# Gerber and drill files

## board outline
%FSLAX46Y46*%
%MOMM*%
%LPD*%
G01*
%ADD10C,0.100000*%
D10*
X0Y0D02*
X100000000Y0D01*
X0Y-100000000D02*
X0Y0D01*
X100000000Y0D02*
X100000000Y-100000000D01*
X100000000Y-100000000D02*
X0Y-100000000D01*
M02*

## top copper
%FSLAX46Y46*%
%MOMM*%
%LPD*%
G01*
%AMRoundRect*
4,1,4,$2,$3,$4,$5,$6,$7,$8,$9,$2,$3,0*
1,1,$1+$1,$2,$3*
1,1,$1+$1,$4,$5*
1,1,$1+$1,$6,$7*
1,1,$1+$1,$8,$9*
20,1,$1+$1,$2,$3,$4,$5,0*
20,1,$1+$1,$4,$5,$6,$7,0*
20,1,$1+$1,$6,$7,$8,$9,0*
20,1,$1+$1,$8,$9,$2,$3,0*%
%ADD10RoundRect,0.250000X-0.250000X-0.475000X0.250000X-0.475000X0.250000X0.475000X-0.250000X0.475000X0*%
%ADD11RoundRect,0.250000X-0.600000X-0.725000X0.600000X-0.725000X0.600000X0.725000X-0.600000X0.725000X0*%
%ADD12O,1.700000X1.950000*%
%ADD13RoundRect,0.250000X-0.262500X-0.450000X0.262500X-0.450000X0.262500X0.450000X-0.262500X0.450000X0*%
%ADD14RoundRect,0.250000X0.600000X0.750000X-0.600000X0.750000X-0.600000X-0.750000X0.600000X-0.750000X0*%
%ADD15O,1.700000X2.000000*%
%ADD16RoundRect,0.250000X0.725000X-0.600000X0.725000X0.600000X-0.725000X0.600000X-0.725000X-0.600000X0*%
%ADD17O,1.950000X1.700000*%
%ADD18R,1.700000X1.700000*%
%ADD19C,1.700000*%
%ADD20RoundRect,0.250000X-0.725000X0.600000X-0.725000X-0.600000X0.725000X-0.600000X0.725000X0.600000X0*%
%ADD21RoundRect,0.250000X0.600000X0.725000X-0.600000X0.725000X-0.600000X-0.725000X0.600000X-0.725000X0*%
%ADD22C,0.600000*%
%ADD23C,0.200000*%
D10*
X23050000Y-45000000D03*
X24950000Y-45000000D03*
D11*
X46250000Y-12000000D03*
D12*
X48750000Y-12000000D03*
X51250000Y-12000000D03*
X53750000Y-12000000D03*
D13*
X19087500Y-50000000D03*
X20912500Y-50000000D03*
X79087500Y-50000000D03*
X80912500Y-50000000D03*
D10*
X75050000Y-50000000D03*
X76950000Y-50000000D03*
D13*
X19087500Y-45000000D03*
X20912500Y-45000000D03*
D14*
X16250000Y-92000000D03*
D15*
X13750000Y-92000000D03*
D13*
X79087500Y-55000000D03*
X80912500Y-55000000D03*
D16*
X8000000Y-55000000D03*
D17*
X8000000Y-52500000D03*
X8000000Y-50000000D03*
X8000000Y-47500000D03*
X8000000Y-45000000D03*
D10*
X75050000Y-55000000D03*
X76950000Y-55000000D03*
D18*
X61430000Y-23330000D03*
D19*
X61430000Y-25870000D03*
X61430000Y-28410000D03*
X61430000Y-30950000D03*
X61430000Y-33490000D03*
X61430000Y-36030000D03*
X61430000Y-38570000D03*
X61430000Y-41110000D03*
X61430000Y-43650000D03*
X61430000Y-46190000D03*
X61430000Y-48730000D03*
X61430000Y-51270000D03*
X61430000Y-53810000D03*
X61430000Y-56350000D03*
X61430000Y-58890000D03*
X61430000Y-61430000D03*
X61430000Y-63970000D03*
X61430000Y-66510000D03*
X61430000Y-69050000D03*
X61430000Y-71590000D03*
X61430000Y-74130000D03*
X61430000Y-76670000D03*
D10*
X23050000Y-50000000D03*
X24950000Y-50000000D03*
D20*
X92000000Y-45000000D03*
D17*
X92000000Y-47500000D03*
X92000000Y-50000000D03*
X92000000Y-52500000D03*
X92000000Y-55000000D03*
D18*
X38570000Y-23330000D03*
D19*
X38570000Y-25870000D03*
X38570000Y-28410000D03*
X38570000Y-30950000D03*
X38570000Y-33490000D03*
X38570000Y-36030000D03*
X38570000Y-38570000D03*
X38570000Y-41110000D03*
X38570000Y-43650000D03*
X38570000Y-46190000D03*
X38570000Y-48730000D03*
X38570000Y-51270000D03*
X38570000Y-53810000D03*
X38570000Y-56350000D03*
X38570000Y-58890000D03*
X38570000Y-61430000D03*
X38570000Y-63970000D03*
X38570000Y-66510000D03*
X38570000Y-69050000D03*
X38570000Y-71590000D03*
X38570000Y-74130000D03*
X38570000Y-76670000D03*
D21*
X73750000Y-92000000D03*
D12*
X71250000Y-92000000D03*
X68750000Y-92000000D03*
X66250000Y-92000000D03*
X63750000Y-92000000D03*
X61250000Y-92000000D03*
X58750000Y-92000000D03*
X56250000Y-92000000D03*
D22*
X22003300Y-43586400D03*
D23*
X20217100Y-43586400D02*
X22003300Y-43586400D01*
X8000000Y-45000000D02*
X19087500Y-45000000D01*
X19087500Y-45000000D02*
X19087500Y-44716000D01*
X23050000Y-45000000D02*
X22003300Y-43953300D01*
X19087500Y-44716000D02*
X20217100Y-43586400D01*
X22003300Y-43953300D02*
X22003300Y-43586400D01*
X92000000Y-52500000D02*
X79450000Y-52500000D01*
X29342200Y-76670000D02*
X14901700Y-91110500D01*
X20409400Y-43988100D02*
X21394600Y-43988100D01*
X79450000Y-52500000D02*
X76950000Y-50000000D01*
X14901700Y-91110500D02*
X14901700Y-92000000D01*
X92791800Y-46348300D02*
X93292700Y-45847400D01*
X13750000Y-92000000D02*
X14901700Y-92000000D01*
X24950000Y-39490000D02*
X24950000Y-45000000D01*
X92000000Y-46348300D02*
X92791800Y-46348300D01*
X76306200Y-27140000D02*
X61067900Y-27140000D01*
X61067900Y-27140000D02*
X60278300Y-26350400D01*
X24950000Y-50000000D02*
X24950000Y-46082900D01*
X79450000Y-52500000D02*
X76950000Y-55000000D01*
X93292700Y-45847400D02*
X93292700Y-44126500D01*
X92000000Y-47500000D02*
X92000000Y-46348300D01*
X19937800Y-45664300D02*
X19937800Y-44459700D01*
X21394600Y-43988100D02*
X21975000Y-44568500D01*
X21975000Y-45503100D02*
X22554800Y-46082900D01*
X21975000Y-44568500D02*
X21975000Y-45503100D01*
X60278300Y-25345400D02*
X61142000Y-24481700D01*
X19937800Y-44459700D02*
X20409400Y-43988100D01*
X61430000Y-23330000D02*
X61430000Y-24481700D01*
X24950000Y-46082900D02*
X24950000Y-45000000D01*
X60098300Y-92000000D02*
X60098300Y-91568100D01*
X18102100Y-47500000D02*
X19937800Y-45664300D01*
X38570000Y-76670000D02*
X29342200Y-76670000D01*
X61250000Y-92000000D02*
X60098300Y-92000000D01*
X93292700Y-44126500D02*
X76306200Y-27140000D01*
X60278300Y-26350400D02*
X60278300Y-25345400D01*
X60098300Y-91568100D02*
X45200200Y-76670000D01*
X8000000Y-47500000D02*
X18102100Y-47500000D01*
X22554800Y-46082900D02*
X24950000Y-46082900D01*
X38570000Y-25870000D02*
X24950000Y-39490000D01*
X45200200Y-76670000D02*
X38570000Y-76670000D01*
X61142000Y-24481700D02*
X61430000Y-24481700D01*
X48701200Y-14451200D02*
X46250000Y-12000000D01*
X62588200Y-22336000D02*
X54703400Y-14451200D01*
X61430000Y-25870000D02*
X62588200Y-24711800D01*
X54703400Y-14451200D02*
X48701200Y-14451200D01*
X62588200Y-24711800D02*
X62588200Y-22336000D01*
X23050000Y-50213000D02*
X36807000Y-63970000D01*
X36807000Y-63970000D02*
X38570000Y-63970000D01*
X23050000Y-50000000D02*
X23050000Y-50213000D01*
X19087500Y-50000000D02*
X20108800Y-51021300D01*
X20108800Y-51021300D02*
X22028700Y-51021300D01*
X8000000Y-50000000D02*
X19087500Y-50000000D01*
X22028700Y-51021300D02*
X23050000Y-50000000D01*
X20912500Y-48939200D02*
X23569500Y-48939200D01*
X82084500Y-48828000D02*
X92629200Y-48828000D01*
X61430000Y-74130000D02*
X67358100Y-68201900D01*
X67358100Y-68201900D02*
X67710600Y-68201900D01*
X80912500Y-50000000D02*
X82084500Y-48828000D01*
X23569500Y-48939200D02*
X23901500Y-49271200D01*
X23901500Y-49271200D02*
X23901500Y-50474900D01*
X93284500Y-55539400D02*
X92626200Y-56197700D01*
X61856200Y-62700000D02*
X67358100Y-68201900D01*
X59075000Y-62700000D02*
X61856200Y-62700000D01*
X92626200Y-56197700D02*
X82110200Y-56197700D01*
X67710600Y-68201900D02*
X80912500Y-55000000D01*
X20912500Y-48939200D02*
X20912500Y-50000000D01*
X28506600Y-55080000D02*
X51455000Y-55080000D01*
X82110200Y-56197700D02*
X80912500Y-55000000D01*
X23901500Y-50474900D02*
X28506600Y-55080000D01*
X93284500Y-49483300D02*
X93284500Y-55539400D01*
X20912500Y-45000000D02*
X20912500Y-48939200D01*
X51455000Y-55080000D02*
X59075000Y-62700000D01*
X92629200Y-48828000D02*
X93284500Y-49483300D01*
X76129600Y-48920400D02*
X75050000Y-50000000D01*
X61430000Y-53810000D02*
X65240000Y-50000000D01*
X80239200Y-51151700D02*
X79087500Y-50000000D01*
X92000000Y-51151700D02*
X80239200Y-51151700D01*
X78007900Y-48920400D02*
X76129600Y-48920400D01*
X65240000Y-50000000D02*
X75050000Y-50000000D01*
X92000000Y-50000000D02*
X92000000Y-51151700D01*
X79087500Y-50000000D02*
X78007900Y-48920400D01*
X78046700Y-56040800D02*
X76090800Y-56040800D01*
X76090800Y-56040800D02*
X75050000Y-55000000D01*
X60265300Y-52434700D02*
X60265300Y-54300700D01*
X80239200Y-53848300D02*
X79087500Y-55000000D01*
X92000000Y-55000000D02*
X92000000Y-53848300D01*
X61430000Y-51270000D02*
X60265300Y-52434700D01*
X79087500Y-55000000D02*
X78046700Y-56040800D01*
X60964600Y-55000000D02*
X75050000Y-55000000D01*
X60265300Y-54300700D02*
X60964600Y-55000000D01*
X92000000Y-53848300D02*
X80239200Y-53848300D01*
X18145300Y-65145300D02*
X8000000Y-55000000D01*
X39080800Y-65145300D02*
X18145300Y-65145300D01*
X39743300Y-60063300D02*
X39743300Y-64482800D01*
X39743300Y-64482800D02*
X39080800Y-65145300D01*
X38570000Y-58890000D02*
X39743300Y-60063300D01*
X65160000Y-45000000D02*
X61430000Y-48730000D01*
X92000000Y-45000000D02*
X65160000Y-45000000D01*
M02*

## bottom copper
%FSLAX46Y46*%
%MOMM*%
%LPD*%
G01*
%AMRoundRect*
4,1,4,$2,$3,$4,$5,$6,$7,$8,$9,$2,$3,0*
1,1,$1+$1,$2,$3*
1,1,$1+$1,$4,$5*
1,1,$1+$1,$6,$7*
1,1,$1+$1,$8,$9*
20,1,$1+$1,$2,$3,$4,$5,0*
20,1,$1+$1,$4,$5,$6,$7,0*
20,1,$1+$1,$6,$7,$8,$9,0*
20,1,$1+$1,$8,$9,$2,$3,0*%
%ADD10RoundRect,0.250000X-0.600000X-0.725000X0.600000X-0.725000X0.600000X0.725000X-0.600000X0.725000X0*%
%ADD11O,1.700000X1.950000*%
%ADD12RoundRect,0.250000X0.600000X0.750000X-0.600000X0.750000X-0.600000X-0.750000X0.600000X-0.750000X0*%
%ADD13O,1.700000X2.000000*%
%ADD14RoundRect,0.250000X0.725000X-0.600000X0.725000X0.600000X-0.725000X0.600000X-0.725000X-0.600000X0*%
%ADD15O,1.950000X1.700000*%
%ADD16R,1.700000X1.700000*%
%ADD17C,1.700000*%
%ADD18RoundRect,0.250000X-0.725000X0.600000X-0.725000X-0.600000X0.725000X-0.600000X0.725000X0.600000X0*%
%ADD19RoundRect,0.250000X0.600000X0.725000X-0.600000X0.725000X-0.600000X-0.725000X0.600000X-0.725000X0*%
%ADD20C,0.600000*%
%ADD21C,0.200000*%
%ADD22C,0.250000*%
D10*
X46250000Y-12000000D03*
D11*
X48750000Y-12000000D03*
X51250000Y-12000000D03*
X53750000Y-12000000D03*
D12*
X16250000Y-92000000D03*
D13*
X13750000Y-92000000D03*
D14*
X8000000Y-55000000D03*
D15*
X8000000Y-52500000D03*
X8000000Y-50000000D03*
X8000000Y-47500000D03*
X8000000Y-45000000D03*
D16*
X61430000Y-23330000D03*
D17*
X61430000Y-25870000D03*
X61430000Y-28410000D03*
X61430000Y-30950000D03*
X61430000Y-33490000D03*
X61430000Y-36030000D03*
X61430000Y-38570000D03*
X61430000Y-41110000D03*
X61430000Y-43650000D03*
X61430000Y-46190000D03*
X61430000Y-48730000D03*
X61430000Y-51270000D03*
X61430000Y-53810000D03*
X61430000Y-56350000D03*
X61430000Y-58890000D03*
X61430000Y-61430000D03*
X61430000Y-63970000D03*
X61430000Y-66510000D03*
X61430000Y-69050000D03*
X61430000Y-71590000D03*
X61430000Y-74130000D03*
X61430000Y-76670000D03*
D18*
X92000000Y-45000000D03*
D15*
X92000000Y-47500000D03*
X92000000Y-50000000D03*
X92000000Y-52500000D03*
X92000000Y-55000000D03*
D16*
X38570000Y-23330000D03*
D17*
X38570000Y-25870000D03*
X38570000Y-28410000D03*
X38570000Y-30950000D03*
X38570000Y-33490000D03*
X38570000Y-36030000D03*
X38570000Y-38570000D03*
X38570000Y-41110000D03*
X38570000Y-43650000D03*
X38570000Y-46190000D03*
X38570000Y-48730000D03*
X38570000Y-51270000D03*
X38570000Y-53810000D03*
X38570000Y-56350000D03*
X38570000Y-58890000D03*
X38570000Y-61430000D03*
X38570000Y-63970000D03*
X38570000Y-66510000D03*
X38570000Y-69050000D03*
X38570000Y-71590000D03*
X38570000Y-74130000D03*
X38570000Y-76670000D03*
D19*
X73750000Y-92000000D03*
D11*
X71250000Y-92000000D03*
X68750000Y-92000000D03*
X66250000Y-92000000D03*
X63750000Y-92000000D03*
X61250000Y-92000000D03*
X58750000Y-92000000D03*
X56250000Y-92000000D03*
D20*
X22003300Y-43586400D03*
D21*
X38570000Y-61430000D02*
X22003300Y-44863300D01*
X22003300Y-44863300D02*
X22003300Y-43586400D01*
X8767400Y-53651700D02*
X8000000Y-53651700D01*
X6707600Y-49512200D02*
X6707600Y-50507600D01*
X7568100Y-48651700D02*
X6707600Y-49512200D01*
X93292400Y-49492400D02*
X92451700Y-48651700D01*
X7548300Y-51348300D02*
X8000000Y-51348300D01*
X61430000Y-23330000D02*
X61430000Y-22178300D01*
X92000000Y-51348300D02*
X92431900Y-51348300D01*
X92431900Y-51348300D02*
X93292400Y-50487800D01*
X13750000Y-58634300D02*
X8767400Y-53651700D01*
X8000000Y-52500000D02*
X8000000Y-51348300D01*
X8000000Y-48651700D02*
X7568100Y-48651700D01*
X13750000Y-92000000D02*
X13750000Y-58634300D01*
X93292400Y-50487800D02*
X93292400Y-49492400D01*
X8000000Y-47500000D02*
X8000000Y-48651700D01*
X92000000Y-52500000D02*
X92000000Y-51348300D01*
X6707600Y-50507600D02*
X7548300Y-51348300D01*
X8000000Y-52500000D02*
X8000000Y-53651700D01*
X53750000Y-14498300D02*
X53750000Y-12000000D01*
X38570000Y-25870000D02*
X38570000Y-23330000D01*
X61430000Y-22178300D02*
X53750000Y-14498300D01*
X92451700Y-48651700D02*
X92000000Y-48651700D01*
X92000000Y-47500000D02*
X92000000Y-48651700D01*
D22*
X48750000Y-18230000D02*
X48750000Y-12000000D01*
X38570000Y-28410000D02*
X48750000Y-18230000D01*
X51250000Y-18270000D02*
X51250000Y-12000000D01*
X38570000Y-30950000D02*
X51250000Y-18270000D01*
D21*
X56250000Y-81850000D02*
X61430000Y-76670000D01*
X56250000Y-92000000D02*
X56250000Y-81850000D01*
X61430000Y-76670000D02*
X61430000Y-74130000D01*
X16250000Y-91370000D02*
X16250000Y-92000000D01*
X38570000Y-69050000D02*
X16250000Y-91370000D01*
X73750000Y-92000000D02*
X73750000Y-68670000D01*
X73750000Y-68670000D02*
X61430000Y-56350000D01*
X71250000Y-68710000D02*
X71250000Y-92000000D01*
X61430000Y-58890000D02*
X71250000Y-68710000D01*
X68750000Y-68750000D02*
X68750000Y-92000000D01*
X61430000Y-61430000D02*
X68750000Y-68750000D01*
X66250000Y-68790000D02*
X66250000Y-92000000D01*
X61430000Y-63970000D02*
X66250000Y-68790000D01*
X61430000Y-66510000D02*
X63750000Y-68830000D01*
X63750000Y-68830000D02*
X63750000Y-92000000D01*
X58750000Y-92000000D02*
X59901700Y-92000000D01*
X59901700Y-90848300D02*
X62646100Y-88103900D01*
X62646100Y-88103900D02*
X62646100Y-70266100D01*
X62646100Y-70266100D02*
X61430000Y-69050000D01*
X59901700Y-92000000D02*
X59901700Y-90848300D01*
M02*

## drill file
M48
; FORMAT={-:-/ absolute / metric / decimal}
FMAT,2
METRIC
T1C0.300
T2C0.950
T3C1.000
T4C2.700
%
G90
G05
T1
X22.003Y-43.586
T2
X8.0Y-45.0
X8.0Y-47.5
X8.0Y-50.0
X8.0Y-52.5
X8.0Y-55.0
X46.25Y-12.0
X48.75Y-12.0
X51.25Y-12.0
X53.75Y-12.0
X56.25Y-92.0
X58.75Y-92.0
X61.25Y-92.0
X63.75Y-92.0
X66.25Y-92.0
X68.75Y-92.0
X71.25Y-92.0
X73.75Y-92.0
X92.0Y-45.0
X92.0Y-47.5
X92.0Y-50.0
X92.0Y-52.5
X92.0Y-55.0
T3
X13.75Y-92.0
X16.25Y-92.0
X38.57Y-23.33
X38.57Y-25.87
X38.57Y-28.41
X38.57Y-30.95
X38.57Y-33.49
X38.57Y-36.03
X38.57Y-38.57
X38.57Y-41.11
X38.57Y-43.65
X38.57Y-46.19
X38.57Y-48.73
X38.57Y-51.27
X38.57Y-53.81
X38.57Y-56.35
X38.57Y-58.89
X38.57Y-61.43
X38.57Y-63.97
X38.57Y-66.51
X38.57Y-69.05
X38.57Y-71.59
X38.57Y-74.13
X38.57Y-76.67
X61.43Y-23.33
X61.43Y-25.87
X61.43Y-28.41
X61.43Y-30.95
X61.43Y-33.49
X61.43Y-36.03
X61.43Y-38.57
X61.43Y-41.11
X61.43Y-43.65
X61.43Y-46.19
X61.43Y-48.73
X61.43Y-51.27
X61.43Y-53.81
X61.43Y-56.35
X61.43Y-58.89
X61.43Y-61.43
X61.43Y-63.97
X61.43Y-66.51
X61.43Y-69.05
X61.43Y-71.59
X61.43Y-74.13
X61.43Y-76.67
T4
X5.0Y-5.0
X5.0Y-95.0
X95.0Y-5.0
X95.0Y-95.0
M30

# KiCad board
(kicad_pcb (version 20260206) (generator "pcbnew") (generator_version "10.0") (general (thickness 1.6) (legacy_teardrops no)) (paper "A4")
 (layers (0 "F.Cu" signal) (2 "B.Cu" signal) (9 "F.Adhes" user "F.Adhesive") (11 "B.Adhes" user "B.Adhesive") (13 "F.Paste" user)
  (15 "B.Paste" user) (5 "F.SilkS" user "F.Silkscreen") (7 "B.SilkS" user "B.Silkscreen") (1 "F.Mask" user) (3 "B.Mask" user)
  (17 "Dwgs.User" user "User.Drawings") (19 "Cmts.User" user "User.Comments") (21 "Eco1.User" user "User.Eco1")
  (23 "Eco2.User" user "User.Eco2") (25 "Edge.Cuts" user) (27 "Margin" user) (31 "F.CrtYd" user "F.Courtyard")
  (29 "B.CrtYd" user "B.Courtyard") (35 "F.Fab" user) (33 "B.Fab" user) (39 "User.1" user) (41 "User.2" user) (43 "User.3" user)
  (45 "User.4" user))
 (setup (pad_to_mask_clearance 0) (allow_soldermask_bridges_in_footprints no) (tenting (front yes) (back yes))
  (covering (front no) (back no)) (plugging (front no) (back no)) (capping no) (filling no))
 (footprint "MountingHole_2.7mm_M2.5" (layer "F.Cu") (at 95 5)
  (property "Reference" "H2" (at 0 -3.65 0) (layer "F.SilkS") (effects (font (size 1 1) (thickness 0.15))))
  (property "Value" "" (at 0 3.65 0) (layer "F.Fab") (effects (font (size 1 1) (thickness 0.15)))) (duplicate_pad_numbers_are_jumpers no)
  (pad "" np_thru_hole circle (at 0 0) (size 2.7 2.7) (drill 2.7) (layers "*.Cu" "*.Mask")))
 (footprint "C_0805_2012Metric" (layer "F.Cu") (at 24 45)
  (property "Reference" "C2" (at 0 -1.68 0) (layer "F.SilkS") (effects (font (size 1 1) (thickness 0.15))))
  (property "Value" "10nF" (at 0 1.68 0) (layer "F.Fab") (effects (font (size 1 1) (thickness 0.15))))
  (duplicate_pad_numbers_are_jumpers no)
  (pad "1" smd roundrect (at -0.95 0) (size 1 1.45) (layers "F.Cu" "F.Mask" "F.Paste") (roundrect_rratio 0.25) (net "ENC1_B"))
  (pad "2" smd roundrect (at 0.95 0) (size 1 1.45) (layers "F.Cu" "F.Mask" "F.Paste") (roundrect_rratio 0.25) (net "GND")))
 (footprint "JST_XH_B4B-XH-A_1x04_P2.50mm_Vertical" (layer "F.Cu") (at 46.25 12)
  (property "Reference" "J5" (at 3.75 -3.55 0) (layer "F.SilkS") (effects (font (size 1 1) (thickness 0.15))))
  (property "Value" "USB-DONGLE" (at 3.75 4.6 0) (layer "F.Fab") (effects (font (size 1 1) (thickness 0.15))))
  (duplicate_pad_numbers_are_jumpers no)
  (pad "1" thru_hole roundrect (at 0 0) (size 1.7 1.95) (drill 0.95) (layers "*.Cu" "*.Mask") (remove_unused_layers no)
   (roundrect_rratio 0.147059) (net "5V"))
  (pad "2" thru_hole oval (at 2.5 0) (size 1.7 1.95) (drill 0.95) (layers "*.Cu" "*.Mask") (remove_unused_layers no) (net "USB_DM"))
  (pad "3" thru_hole oval (at 5 0) (size 1.7 1.95) (drill 0.95) (layers "*.Cu" "*.Mask") (remove_unused_layers no) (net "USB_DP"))
  (pad "4" thru_hole oval (at 7.5 0) (size 1.7 1.95) (drill 0.95) (layers "*.Cu" "*.Mask") (remove_unused_layers no) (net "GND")))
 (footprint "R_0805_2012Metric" (layer "F.Cu") (at 20 50)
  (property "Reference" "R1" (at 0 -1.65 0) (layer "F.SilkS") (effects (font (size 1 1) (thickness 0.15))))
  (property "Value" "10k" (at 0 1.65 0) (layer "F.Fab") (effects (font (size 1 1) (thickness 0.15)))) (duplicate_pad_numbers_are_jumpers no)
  (pad "1" smd roundrect (at -0.9125 0) (size 1.025 1.4) (layers "F.Cu" "F.Mask" "F.Paste") (roundrect_rratio 0.243902) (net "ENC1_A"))
  (pad "2" smd roundrect (at 0.9125 0) (size 1.025 1.4) (layers "F.Cu" "F.Mask" "F.Paste") (roundrect_rratio 0.243902) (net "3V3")))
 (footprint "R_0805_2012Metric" (layer "F.Cu") (at 80 50)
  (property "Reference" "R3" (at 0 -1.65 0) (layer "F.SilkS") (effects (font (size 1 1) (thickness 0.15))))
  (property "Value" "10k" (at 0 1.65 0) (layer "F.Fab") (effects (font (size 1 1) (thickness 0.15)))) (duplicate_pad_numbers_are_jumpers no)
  (pad "1" smd roundrect (at -0.9125 0) (size 1.025 1.4) (layers "F.Cu" "F.Mask" "F.Paste") (roundrect_rratio 0.243902) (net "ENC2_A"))
  (pad "2" smd roundrect (at 0.9125 0) (size 1.025 1.4) (layers "F.Cu" "F.Mask" "F.Paste") (roundrect_rratio 0.243902) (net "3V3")))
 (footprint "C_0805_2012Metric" (layer "F.Cu") (at 76 50)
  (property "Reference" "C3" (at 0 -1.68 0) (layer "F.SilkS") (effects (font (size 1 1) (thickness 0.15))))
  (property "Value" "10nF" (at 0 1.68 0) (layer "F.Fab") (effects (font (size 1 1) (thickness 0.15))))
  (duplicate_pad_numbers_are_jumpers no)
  (pad "1" smd roundrect (at -0.95 0) (size 1 1.45) (layers "F.Cu" "F.Mask" "F.Paste") (roundrect_rratio 0.25) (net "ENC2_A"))
  (pad "2" smd roundrect (at 0.95 0) (size 1 1.45) (layers "F.Cu" "F.Mask" "F.Paste") (roundrect_rratio 0.25) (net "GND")))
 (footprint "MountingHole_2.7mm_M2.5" (layer "F.Cu") (at 95 95)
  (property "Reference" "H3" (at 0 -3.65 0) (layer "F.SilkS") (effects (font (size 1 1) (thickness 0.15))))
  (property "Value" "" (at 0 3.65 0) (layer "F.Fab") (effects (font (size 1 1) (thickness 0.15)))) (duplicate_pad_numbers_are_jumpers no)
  (pad "" np_thru_hole circle (at 0 0) (size 2.7 2.7) (drill 2.7) (layers "*.Cu" "*.Mask")))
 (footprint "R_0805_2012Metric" (layer "F.Cu") (at 20 45)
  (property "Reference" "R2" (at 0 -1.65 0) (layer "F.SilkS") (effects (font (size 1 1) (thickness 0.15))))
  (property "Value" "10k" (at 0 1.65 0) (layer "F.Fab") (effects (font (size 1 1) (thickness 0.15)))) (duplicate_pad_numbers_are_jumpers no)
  (pad "1" smd roundrect (at -0.9125 0) (size 1.025 1.4) (layers "F.Cu" "F.Mask" "F.Paste") (roundrect_rratio 0.243902) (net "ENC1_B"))
  (pad "2" smd roundrect (at 0.9125 0) (size 1.025 1.4) (layers "F.Cu" "F.Mask" "F.Paste") (roundrect_rratio 0.243902) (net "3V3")))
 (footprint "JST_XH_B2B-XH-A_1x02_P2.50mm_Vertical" (layer "F.Cu") (at 16.25 92 180)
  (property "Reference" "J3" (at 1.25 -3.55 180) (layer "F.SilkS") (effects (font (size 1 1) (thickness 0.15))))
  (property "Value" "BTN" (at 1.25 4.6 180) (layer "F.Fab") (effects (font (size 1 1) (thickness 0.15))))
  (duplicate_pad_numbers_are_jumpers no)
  (pad "1" thru_hole roundrect (at 0 0 180) (size 1.7 2) (drill 1) (layers "*.Cu" "*.Mask") (remove_unused_layers no)
   (roundrect_rratio 0.147059) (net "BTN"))
  (pad "2" thru_hole oval (at 2.5 0 180) (size 1.7 2) (drill 1) (layers "*.Cu" "*.Mask") (remove_unused_layers no) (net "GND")))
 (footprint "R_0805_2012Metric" (layer "F.Cu") (at 80 55)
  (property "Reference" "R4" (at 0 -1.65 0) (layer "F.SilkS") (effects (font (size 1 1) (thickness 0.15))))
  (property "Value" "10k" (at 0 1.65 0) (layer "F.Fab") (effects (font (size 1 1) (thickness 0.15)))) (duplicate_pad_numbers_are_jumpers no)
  (pad "1" smd roundrect (at -0.9125 0) (size 1.025 1.4) (layers "F.Cu" "F.Mask" "F.Paste") (roundrect_rratio 0.243902) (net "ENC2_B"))
  (pad "2" smd roundrect (at 0.9125 0) (size 1.025 1.4) (layers "F.Cu" "F.Mask" "F.Paste") (roundrect_rratio 0.243902) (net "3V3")))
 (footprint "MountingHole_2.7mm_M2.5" (layer "F.Cu") (at 5 5)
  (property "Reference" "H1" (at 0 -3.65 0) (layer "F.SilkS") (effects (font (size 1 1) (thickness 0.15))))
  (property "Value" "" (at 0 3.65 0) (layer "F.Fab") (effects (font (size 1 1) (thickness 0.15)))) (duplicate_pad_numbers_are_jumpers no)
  (pad "" np_thru_hole circle (at 0 0) (size 2.7 2.7) (drill 2.7) (layers "*.Cu" "*.Mask")))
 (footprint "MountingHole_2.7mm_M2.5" (layer "F.Cu") (at 5 95)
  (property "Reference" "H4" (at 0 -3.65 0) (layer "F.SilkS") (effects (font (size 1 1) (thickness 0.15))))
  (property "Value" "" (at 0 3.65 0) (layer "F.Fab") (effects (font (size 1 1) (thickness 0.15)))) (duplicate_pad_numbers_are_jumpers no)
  (pad "" np_thru_hole circle (at 0 0) (size 2.7 2.7) (drill 2.7) (layers "*.Cu" "*.Mask")))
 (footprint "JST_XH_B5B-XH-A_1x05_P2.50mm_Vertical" (layer "F.Cu") (at 8 55 90)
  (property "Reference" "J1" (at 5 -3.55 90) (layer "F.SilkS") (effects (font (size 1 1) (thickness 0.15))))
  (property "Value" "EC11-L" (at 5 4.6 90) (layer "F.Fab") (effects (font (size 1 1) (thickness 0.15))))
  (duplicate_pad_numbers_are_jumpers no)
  (pad "1" thru_hole roundrect (at 0 0 90) (size 1.7 1.95) (drill 0.95) (layers "*.Cu" "*.Mask") (remove_unused_layers no)
   (roundrect_rratio 0.147059) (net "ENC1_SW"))
  (pad "2" thru_hole oval (at 2.5 0 90) (size 1.7 1.95) (drill 0.95) (layers "*.Cu" "*.Mask") (remove_unused_layers no) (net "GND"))
  (pad "3" thru_hole oval (at 5 0 90) (size 1.7 1.95) (drill 0.95) (layers "*.Cu" "*.Mask") (remove_unused_layers no) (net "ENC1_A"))
  (pad "4" thru_hole oval (at 7.5 0 90) (size 1.7 1.95) (drill 0.95) (layers "*.Cu" "*.Mask") (remove_unused_layers no) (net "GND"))
  (pad "5" thru_hole oval (at 10 0 90) (size 1.7 1.95) (drill 0.95) (layers "*.Cu" "*.Mask") (remove_unused_layers no) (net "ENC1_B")))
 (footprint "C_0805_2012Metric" (layer "F.Cu") (at 76 55)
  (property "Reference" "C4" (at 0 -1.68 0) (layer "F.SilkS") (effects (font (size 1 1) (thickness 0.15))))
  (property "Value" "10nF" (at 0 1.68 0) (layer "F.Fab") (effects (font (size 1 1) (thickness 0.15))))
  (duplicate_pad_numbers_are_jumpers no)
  (pad "1" smd roundrect (at -0.95 0) (size 1 1.45) (layers "F.Cu" "F.Mask" "F.Paste") (roundrect_rratio 0.25) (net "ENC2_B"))
  (pad "2" smd roundrect (at 0.95 0) (size 1 1.45) (layers "F.Cu" "F.Mask" "F.Paste") (roundrect_rratio 0.25) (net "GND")))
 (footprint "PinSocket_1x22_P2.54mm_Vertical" (layer "F.Cu") (at 61.43 23.33)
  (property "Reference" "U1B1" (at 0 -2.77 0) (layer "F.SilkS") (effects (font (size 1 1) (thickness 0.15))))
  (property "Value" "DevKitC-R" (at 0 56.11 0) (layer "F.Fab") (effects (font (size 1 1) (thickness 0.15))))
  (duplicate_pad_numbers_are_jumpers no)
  (pad "1" thru_hole rect (at 0 0) (size 1.7 1.7) (drill 1) (layers "*.Cu" "*.Mask") (remove_unused_layers no) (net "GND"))
  (pad "2" thru_hole circle (at 0 2.54) (size 1.7 1.7) (drill 1) (layers "*.Cu" "*.Mask") (remove_unused_layers no) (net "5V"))
  (pad "3" thru_hole circle (at 0 5.08) (size 1.7 1.7) (drill 1) (layers "*.Cu" "*.Mask") (remove_unused_layers no))
  (pad "4" thru_hole circle (at 0 7.62) (size 1.7 1.7) (drill 1) (layers "*.Cu" "*.Mask") (remove_unused_layers no))
  (pad "5" thru_hole circle (at 0 10.16) (size 1.7 1.7) (drill 1) (layers "*.Cu" "*.Mask") (remove_unused_layers no))
  (pad "6" thru_hole circle (at 0 12.7) (size 1.7 1.7) (drill 1) (layers "*.Cu" "*.Mask") (remove_unused_layers no))
  (pad "7" thru_hole circle (at 0 15.24) (size 1.7 1.7) (drill 1) (layers "*.Cu" "*.Mask") (remove_unused_layers no))
  (pad "8" thru_hole circle (at 0 17.78) (size 1.7 1.7) (drill 1) (layers "*.Cu" "*.Mask") (remove_unused_layers no))
  (pad "9" thru_hole circle (at 0 20.32) (size 1.7 1.7) (drill 1) (layers "*.Cu" "*.Mask") (remove_unused_layers no))
  (pad "10" thru_hole circle (at 0 22.86) (size 1.7 1.7) (drill 1) (layers "*.Cu" "*.Mask") (remove_unused_layers no))
  (pad "11" thru_hole circle (at 0 25.4) (size 1.7 1.7) (drill 1) (layers "*.Cu" "*.Mask") (remove_unused_layers no) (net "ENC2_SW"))
  (pad "12" thru_hole circle (at 0 27.94) (size 1.7 1.7) (drill 1) (layers "*.Cu" "*.Mask") (remove_unused_layers no) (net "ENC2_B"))
  (pad "13" thru_hole circle (at 0 30.48) (size 1.7 1.7) (drill 1) (layers "*.Cu" "*.Mask") (remove_unused_layers no) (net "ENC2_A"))
  (pad "14" thru_hole circle (at 0 33.02) (size 1.7 1.7) (drill 1) (layers "*.Cu" "*.Mask") (remove_unused_layers no) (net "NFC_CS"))
  (pad "15" thru_hole circle (at 0 35.56) (size 1.7 1.7) (drill 1) (layers "*.Cu" "*.Mask") (remove_unused_layers no) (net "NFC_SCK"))
  (pad "16" thru_hole circle (at 0 38.1) (size 1.7 1.7) (drill 1) (layers "*.Cu" "*.Mask") (remove_unused_layers no) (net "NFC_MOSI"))
  (pad "17" thru_hole circle (at 0 40.64) (size 1.7 1.7) (drill 1) (layers "*.Cu" "*.Mask") (remove_unused_layers no) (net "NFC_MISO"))
  (pad "18" thru_hole circle (at 0 43.18) (size 1.7 1.7) (drill 1) (layers "*.Cu" "*.Mask") (remove_unused_layers no) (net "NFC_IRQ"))
  (pad "19" thru_hole circle (at 0 45.72) (size 1.7 1.7) (drill 1) (layers "*.Cu" "*.Mask") (remove_unused_layers no) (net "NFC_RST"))
  (pad "20" thru_hole circle (at 0 48.26) (size 1.7 1.7) (drill 1) (layers "*.Cu" "*.Mask") (remove_unused_layers no))
  (pad "21" thru_hole circle (at 0 50.8) (size 1.7 1.7) (drill 1) (layers "*.Cu" "*.Mask") (remove_unused_layers no) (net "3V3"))
  (pad "22" thru_hole circle (at 0 53.34) (size 1.7 1.7) (drill 1) (layers "*.Cu" "*.Mask") (remove_unused_layers no) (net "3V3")))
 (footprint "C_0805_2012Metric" (layer "F.Cu") (at 24 50)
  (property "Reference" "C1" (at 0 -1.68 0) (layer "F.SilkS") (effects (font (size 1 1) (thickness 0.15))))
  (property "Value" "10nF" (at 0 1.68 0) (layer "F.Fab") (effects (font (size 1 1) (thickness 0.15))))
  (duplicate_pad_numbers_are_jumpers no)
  (pad "1" smd roundrect (at -0.95 0) (size 1 1.45) (layers "F.Cu" "F.Mask" "F.Paste") (roundrect_rratio 0.25) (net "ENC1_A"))
  (pad "2" smd roundrect (at 0.95 0) (size 1 1.45) (layers "F.Cu" "F.Mask" "F.Paste") (roundrect_rratio 0.25) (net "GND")))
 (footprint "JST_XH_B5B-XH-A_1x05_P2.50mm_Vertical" (layer "F.Cu") (at 92 45 -90)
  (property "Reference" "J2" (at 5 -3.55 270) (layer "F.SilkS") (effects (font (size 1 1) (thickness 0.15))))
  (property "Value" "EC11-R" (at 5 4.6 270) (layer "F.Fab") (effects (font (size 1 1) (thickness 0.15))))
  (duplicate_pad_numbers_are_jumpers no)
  (pad "1" thru_hole roundrect (at 0 0 270) (size 1.7 1.95) (drill 0.95) (layers "*.Cu" "*.Mask") (remove_unused_layers no)
   (roundrect_rratio 0.147059) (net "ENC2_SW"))
  (pad "2" thru_hole oval (at 2.5 0 270) (size 1.7 1.95) (drill 0.95) (layers "*.Cu" "*.Mask") (remove_unused_layers no) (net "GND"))
  (pad "3" thru_hole oval (at 5 0 270) (size 1.7 1.95) (drill 0.95) (layers "*.Cu" "*.Mask") (remove_unused_layers no) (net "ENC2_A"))
  (pad "4" thru_hole oval (at 7.5 0 270) (size 1.7 1.95) (drill 0.95) (layers "*.Cu" "*.Mask") (remove_unused_layers no) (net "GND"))
  (pad "5" thru_hole oval (at 10 0 270) (size 1.7 1.95) (drill 0.95) (layers "*.Cu" "*.Mask") (remove_unused_layers no) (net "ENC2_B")))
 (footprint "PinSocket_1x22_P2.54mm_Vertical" (layer "F.Cu") (at 38.57 23.33)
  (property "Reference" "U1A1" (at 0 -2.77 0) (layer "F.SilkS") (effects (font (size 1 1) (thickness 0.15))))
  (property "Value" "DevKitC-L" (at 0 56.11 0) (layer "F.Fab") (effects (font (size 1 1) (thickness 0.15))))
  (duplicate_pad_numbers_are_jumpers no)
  (pad "1" thru_hole rect (at 0 0) (size 1.7 1.7) (drill 1) (layers "*.Cu" "*.Mask") (remove_unused_layers no) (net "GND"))
  (pad "2" thru_hole circle (at 0 2.54) (size 1.7 1.7) (drill 1) (layers "*.Cu" "*.Mask") (remove_unused_layers no) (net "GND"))
  (pad "3" thru_hole circle (at 0 5.08) (size 1.7 1.7) (drill 1) (layers "*.Cu" "*.Mask") (remove_unused_layers no) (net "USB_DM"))
  (pad "4" thru_hole circle (at 0 7.62) (size 1.7 1.7) (drill 1) (layers "*.Cu" "*.Mask") (remove_unused_layers no) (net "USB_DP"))
  (pad "5" thru_hole circle (at 0 10.16) (size 1.7 1.7) (drill 1) (layers "*.Cu" "*.Mask") (remove_unused_layers no))
  (pad "6" thru_hole circle (at 0 12.7) (size 1.7 1.7) (drill 1) (layers "*.Cu" "*.Mask") (remove_unused_layers no))
  (pad "7" thru_hole circle (at 0 15.24) (size 1.7 1.7) (drill 1) (layers "*.Cu" "*.Mask") (remove_unused_layers no))
  (pad "8" thru_hole circle (at 0 17.78) (size 1.7 1.7) (drill 1) (layers "*.Cu" "*.Mask") (remove_unused_layers no))
  (pad "9" thru_hole circle (at 0 20.32) (size 1.7 1.7) (drill 1) (layers "*.Cu" "*.Mask") (remove_unused_layers no))
  (pad "10" thru_hole circle (at 0 22.86) (size 1.7 1.7) (drill 1) (layers "*.Cu" "*.Mask") (remove_unused_layers no))
  (pad "11" thru_hole circle (at 0 25.4) (size 1.7 1.7) (drill 1) (layers "*.Cu" "*.Mask") (remove_unused_layers no))
  (pad "12" thru_hole circle (at 0 27.94) (size 1.7 1.7) (drill 1) (layers "*.Cu" "*.Mask") (remove_unused_layers no))
  (pad "13" thru_hole circle (at 0 30.48) (size 1.7 1.7) (drill 1) (layers "*.Cu" "*.Mask") (remove_unused_layers no))
  (pad "14" thru_hole circle (at 0 33.02) (size 1.7 1.7) (drill 1) (layers "*.Cu" "*.Mask") (remove_unused_layers no))
  (pad "15" thru_hole circle (at 0 35.56) (size 1.7 1.7) (drill 1) (layers "*.Cu" "*.Mask") (remove_unused_layers no) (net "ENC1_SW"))
  (pad "16" thru_hole circle (at 0 38.1) (size 1.7 1.7) (drill 1) (layers "*.Cu" "*.Mask") (remove_unused_layers no) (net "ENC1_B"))
  (pad "17" thru_hole circle (at 0 40.64) (size 1.7 1.7) (drill 1) (layers "*.Cu" "*.Mask") (remove_unused_layers no) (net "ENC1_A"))
  (pad "18" thru_hole circle (at 0 43.18) (size 1.7 1.7) (drill 1) (layers "*.Cu" "*.Mask") (remove_unused_layers no))
  (pad "19" thru_hole circle (at 0 45.72) (size 1.7 1.7) (drill 1) (layers "*.Cu" "*.Mask") (remove_unused_layers no) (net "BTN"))
  (pad "20" thru_hole circle (at 0 48.26) (size 1.7 1.7) (drill 1) (layers "*.Cu" "*.Mask") (remove_unused_layers no))
  (pad "21" thru_hole circle (at 0 50.8) (size 1.7 1.7) (drill 1) (layers "*.Cu" "*.Mask") (remove_unused_layers no))
  (pad "22" thru_hole circle (at 0 53.34) (size 1.7 1.7) (drill 1) (layers "*.Cu" "*.Mask") (remove_unused_layers no) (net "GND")))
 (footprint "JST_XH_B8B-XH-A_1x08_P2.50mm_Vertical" (layer "F.Cu") (at 73.75 92 180)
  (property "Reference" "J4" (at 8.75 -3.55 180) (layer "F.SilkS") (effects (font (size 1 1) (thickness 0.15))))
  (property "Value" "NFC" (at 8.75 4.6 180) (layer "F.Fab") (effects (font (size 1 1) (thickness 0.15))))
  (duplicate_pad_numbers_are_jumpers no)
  (pad "1" thru_hole roundrect (at 0 0 180) (size 1.7 1.95) (drill 0.95) (layers "*.Cu" "*.Mask") (remove_unused_layers no)
   (roundrect_rratio 0.147059) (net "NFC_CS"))
  (pad "2" thru_hole oval (at 2.5 0 180) (size 1.7 1.95) (drill 0.95) (layers "*.Cu" "*.Mask") (remove_unused_layers no) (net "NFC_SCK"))
  (pad "3" thru_hole oval (at 5 0 180) (size 1.7 1.95) (drill 0.95) (layers "*.Cu" "*.Mask") (remove_unused_layers no) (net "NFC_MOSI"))
  (pad "4" thru_hole oval (at 7.5 0 180) (size 1.7 1.95) (drill 0.95) (layers "*.Cu" "*.Mask") (remove_unused_layers no) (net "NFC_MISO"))
  (pad "5" thru_hole oval (at 10 0 180) (size 1.7 1.95) (drill 0.95) (layers "*.Cu" "*.Mask") (remove_unused_layers no) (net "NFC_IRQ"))
  (pad "6" thru_hole oval (at 12.5 0 180) (size 1.7 1.95) (drill 0.95) (layers "*.Cu" "*.Mask") (remove_unused_layers no) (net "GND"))
  (pad "7" thru_hole oval (at 15 0 180) (size 1.7 1.95) (drill 0.95) (layers "*.Cu" "*.Mask") (remove_unused_layers no) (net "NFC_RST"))
  (pad "8" thru_hole oval (at 17.5 0 180) (size 1.7 1.95) (drill 0.95) (layers "*.Cu" "*.Mask") (remove_unused_layers no) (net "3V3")))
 (gr_line (start 0 0) (end 100 0) (stroke (width 0.1) (type default)) (layer "Edge.Cuts"))
 (gr_line (start 0 100) (end 0 0) (stroke (width 0.1) (type default)) (layer "Edge.Cuts"))
 (gr_line (start 100 0) (end 100 100) (stroke (width 0.1) (type default)) (layer "Edge.Cuts"))
 (gr_line (start 100 100) (end 0 100) (stroke (width 0.1) (type default)) (layer "Edge.Cuts"))
 (segment (start 20.2171 43.5864) (end 22.0033 43.5864) (width 0.2) (layer "F.Cu") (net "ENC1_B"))
 (segment (start 8 45) (end 19.0875 45) (width 0.2) (layer "F.Cu") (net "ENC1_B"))
 (segment (start 19.0875 45) (end 19.0875 44.716) (width 0.2) (layer "F.Cu") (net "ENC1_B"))
 (segment (start 23.05 45) (end 22.0033 43.9533) (width 0.2) (layer "F.Cu") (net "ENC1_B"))
 (segment (start 19.0875 44.716) (end 20.2171 43.5864) (width 0.2) (layer "F.Cu") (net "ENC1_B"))
 (segment (start 22.0033 43.9533) (end 22.0033 43.5864) (width 0.2) (layer "F.Cu") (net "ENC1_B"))
 (via (at 22.0033 43.5864) (size 0.6) (drill 0.3) (layers "F.Cu" "B.Cu") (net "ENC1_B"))
 (segment (start 38.57 61.43) (end 22.0033 44.8633) (width 0.2) (layer "B.Cu") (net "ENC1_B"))
 (segment (start 22.0033 44.8633) (end 22.0033 43.5864) (width 0.2) (layer "B.Cu") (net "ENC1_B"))
 (segment (start 92 52.5) (end 79.45 52.5) (width 0.2) (layer "F.Cu") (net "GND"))
 (segment (start 29.3422 76.67) (end 14.9017 91.1105) (width 0.2) (layer "F.Cu") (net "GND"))
 (segment (start 20.4094 43.9881) (end 21.3946 43.9881) (width 0.2) (layer "F.Cu") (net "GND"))
 (segment (start 79.45 52.5) (end 76.95 50) (width 0.2) (layer "F.Cu") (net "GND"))
 (segment (start 14.9017 91.1105) (end 14.9017 92) (width 0.2) (layer "F.Cu") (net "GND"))
 (segment (start 92.7918 46.3483) (end 93.2927 45.8474) (width 0.2) (layer "F.Cu") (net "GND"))
 (segment (start 13.75 92) (end 14.9017 92) (width 0.2) (layer "F.Cu") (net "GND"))
 (segment (start 24.95 39.49) (end 24.95 45) (width 0.2) (layer "F.Cu") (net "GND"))
 (segment (start 92 46.3483) (end 92.7918 46.3483) (width 0.2) (layer "F.Cu") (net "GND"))
 (segment (start 76.3062 27.14) (end 61.0679 27.14) (width 0.2) (layer "F.Cu") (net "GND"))
 (segment (start 61.0679 27.14) (end 60.2783 26.3504) (width 0.2) (layer "F.Cu") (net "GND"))
 (segment (start 24.95 50) (end 24.95 46.0829) (width 0.2) (layer "F.Cu") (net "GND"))
 (segment (start 79.45 52.5) (end 76.95 55) (width 0.2) (layer "F.Cu") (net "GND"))
 (segment (start 93.2927 45.8474) (end 93.2927 44.1265) (width 0.2) (layer "F.Cu") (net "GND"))
 (segment (start 92 47.5) (end 92 46.3483) (width 0.2) (layer "F.Cu") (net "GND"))
 (segment (start 19.9378 45.6643) (end 19.9378 44.4597) (width 0.2) (layer "F.Cu") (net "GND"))
 (segment (start 21.3946 43.9881) (end 21.975 44.5685) (width 0.2) (layer "F.Cu") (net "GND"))
 (segment (start 21.975 45.5031) (end 22.5548 46.0829) (width 0.2) (layer "F.Cu") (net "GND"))
 (segment (start 21.975 44.5685) (end 21.975 45.5031) (width 0.2) (layer "F.Cu") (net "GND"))
 (segment (start 60.2783 25.3454) (end 61.142 24.4817) (width 0.2) (layer "F.Cu") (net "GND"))
 (segment (start 19.9378 44.4597) (end 20.4094 43.9881) (width 0.2) (layer "F.Cu") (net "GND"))
 (segment (start 61.43 23.33) (end 61.43 24.4817) (width 0.2) (layer "F.Cu") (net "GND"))
 (segment (start 24.95 46.0829) (end 24.95 45) (width 0.2) (layer "F.Cu") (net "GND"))
 (segment (start 60.0983 92) (end 60.0983 91.5681) (width 0.2) (layer "F.Cu") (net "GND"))
 (segment (start 18.1021 47.5) (end 19.9378 45.6643) (width 0.2) (layer "F.Cu") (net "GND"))
 (segment (start 38.57 76.67) (end 29.3422 76.67) (width 0.2) (layer "F.Cu") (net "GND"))
 (segment (start 61.25 92) (end 60.0983 92) (width 0.2) (layer "F.Cu") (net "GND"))
 (segment (start 93.2927 44.1265) (end 76.3062 27.14) (width 0.2) (layer "F.Cu") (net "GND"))
 (segment (start 60.2783 26.3504) (end 60.2783 25.3454) (width 0.2) (layer "F.Cu") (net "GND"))
 (segment (start 60.0983 91.5681) (end 45.2002 76.67) (width 0.2) (layer "F.Cu") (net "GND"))
 (segment (start 8 47.5) (end 18.1021 47.5) (width 0.2) (layer "F.Cu") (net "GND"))
 (segment (start 22.5548 46.0829) (end 24.95 46.0829) (width 0.2) (layer "F.Cu") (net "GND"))
 (segment (start 38.57 25.87) (end 24.95 39.49) (width 0.2) (layer "F.Cu") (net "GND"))
 (segment (start 45.2002 76.67) (end 38.57 76.67) (width 0.2) (layer "F.Cu") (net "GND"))
 (segment (start 61.142 24.4817) (end 61.43 24.4817) (width 0.2) (layer "F.Cu") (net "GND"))
 (segment (start 8.7674 53.6517) (end 8 53.6517) (width 0.2) (layer "B.Cu") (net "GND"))
 (segment (start 6.7076 49.5122) (end 6.7076 50.5076) (width 0.2) (layer "B.Cu") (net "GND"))
 (segment (start 7.5681 48.6517) (end 6.7076 49.5122) (width 0.2) (layer "B.Cu") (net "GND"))
 (segment (start 93.2924 49.4924) (end 92.4517 48.6517) (width 0.2) (layer "B.Cu") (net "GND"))
 (segment (start 7.5483 51.3483) (end 8 51.3483) (width 0.2) (layer "B.Cu") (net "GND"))
 (segment (start 61.43 23.33) (end 61.43 22.1783) (width 0.2) (layer "B.Cu") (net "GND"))
 (segment (start 92 51.3483) (end 92.4319 51.3483) (width 0.2) (layer "B.Cu") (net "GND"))
 (segment (start 92.4319 51.3483) (end 93.2924 50.4878) (width 0.2) (layer "B.Cu") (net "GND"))
 (segment (start 13.75 58.6343) (end 8.7674 53.6517) (width 0.2) (layer "B.Cu") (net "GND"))
 (segment (start 8 52.5) (end 8 51.3483) (width 0.2) (layer "B.Cu") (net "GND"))
 (segment (start 8 48.6517) (end 7.5681 48.6517) (width 0.2) (layer "B.Cu") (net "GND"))
 (segment (start 13.75 92) (end 13.75 58.6343) (width 0.2) (layer "B.Cu") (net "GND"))
 (segment (start 93.2924 50.4878) (end 93.2924 49.4924) (width 0.2) (layer "B.Cu") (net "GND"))
 (segment (start 8 47.5) (end 8 48.6517) (width 0.2) (layer "B.Cu") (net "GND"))
 (segment (start 92 52.5) (end 92 51.3483) (width 0.2) (layer "B.Cu") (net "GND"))
 (segment (start 6.7076 50.5076) (end 7.5483 51.3483) (width 0.2) (layer "B.Cu") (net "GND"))
 (segment (start 8 52.5) (end 8 53.6517) (width 0.2) (layer "B.Cu") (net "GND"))
 (segment (start 53.75 14.4983) (end 53.75 12) (width 0.2) (layer "B.Cu") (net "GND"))
 (segment (start 38.57 25.87) (end 38.57 23.33) (width 0.2) (layer "B.Cu") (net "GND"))
 (segment (start 61.43 22.1783) (end 53.75 14.4983) (width 0.2) (layer "B.Cu") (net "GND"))
 (segment (start 92.4517 48.6517) (end 92 48.6517) (width 0.2) (layer "B.Cu") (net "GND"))
 (segment (start 92 47.5) (end 92 48.6517) (width 0.2) (layer "B.Cu") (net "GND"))
 (segment (start 48.7012 14.4512) (end 46.25 12) (width 0.2) (layer "F.Cu") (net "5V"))
 (segment (start 62.5882 22.336) (end 54.7034 14.4512) (width 0.2) (layer "F.Cu") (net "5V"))
 (segment (start 61.43 25.87) (end 62.5882 24.7118) (width 0.2) (layer "F.Cu") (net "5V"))
 (segment (start 54.7034 14.4512) (end 48.7012 14.4512) (width 0.2) (layer "F.Cu") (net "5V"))
 (segment (start 62.5882 24.7118) (end 62.5882 22.336) (width 0.2) (layer "F.Cu") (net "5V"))
 (segment (start 48.75 18.23) (end 48.75 12) (width 0.25) (layer "B.Cu") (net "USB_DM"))
 (segment (start 38.57 28.41) (end 48.75 18.23) (width 0.25) (layer "B.Cu") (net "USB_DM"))
 (segment (start 51.25 18.27) (end 51.25 12) (width 0.25) (layer "B.Cu") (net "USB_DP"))
 (segment (start 38.57 30.95) (end 51.25 18.27) (width 0.25) (layer "B.Cu") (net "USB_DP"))
 (segment (start 23.05 50.213) (end 36.807 63.97) (width 0.2) (layer "F.Cu") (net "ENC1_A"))
 (segment (start 36.807 63.97) (end 38.57 63.97) (width 0.2) (layer "F.Cu") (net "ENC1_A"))
 (segment (start 23.05 50) (end 23.05 50.213) (width 0.2) (layer "F.Cu") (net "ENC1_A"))
 (segment (start 19.0875 50) (end 20.1088 51.0213) (width 0.2) (layer "F.Cu") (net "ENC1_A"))
 (segment (start 20.1088 51.0213) (end 22.0287 51.0213) (width 0.2) (layer "F.Cu") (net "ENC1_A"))
 (segment (start 8 50) (end 19.0875 50) (width 0.2) (layer "F.Cu") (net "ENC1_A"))
 (segment (start 22.0287 51.0213) (end 23.05 50) (width 0.2) (layer "F.Cu") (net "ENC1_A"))
 (segment (start 20.9125 48.9392) (end 23.5695 48.9392) (width 0.2) (layer "F.Cu") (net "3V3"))
 (segment (start 82.0845 48.828) (end 92.6292 48.828) (width 0.2) (layer "F.Cu") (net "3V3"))
 (segment (start 61.43 74.13) (end 67.3581 68.2019) (width 0.2) (layer "F.Cu") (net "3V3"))
 (segment (start 67.3581 68.2019) (end 67.7106 68.2019) (width 0.2) (layer "F.Cu") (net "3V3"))
 (segment (start 80.9125 50) (end 82.0845 48.828) (width 0.2) (layer "F.Cu") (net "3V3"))
 (segment (start 23.5695 48.9392) (end 23.9015 49.2712) (width 0.2) (layer "F.Cu") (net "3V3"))
 (segment (start 23.9015 49.2712) (end 23.9015 50.4749) (width 0.2) (layer "F.Cu") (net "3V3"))
 (segment (start 93.2845 55.5394) (end 92.6262 56.1977) (width 0.2) (layer "F.Cu") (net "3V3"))
 (segment (start 61.8562 62.7) (end 67.3581 68.2019) (width 0.2) (layer "F.Cu") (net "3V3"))
 (segment (start 59.075 62.7) (end 61.8562 62.7) (width 0.2) (layer "F.Cu") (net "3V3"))
 (segment (start 92.6262 56.1977) (end 82.1102 56.1977) (width 0.2) (layer "F.Cu") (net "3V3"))
 (segment (start 67.7106 68.2019) (end 80.9125 55) (width 0.2) (layer "F.Cu") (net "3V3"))
 (segment (start 20.9125 48.9392) (end 20.9125 50) (width 0.2) (layer "F.Cu") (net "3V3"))
 (segment (start 28.5066 55.08) (end 51.455 55.08) (width 0.2) (layer "F.Cu") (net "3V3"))
 (segment (start 82.1102 56.1977) (end 80.9125 55) (width 0.2) (layer "F.Cu") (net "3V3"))
 (segment (start 23.9015 50.4749) (end 28.5066 55.08) (width 0.2) (layer "F.Cu") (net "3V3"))
 (segment (start 93.2845 49.4833) (end 93.2845 55.5394) (width 0.2) (layer "F.Cu") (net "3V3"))
 (segment (start 20.9125 45) (end 20.9125 48.9392) (width 0.2) (layer "F.Cu") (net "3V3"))
 (segment (start 51.455 55.08) (end 59.075 62.7) (width 0.2) (layer "F.Cu") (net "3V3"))
 (segment (start 92.6292 48.828) (end 93.2845 49.4833) (width 0.2) (layer "F.Cu") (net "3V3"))
 (segment (start 56.25 81.85) (end 61.43 76.67) (width 0.2) (layer "B.Cu") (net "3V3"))
 (segment (start 56.25 92) (end 56.25 81.85) (width 0.2) (layer "B.Cu") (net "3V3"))
 (segment (start 61.43 76.67) (end 61.43 74.13) (width 0.2) (layer "B.Cu") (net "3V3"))
 (segment (start 76.1296 48.9204) (end 75.05 50) (width 0.2) (layer "F.Cu") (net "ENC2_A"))
 (segment (start 61.43 53.81) (end 65.24 50) (width 0.2) (layer "F.Cu") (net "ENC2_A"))
 (segment (start 80.2392 51.1517) (end 79.0875 50) (width 0.2) (layer "F.Cu") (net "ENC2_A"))
 (segment (start 92 51.1517) (end 80.2392 51.1517) (width 0.2) (layer "F.Cu") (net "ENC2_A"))
 (segment (start 78.0079 48.9204) (end 76.1296 48.9204) (width 0.2) (layer "F.Cu") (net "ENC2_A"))
 (segment (start 65.24 50) (end 75.05 50) (width 0.2) (layer "F.Cu") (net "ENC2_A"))
 (segment (start 92 50) (end 92 51.1517) (width 0.2) (layer "F.Cu") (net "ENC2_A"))
 (segment (start 79.0875 50) (end 78.0079 48.9204) (width 0.2) (layer "F.Cu") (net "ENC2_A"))
 (segment (start 16.25 91.37) (end 16.25 92) (width 0.2) (layer "B.Cu") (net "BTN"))
 (segment (start 38.57 69.05) (end 16.25 91.37) (width 0.2) (layer "B.Cu") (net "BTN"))
 (segment (start 78.0467 56.0408) (end 76.0908 56.0408) (width 0.2) (layer "F.Cu") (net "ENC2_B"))
 (segment (start 76.0908 56.0408) (end 75.05 55) (width 0.2) (layer "F.Cu") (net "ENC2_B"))
 (segment (start 60.2653 52.4347) (end 60.2653 54.3007) (width 0.2) (layer "F.Cu") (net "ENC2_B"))
 (segment (start 80.2392 53.8483) (end 79.0875 55) (width 0.2) (layer "F.Cu") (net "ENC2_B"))
 (segment (start 92 55) (end 92 53.8483) (width 0.2) (layer "F.Cu") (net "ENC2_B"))
 (segment (start 61.43 51.27) (end 60.2653 52.4347) (width 0.2) (layer "F.Cu") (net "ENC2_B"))
 (segment (start 79.0875 55) (end 78.0467 56.0408) (width 0.2) (layer "F.Cu") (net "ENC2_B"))
 (segment (start 60.9646 55) (end 75.05 55) (width 0.2) (layer "F.Cu") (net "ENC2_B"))
 (segment (start 60.2653 54.3007) (end 60.9646 55) (width 0.2) (layer "F.Cu") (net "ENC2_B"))
 (segment (start 92 53.8483) (end 80.2392 53.8483) (width 0.2) (layer "F.Cu") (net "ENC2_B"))
 (segment (start 18.1453 65.1453) (end 8 55) (width 0.2) (layer "F.Cu") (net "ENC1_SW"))
 (segment (start 39.0808 65.1453) (end 18.1453 65.1453) (width 0.2) (layer "F.Cu") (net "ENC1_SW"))
 (segment (start 39.7433 60.0633) (end 39.7433 64.4828) (width 0.2) (layer "F.Cu") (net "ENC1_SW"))
 (segment (start 39.7433 64.4828) (end 39.0808 65.1453) (width 0.2) (layer "F.Cu") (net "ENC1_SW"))
 (segment (start 38.57 58.89) (end 39.7433 60.0633) (width 0.2) (layer "F.Cu") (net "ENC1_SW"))
 (segment (start 65.16 45) (end 61.43 48.73) (width 0.2) (layer "F.Cu") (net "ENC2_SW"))
 (segment (start 92 45) (end 65.16 45) (width 0.2) (layer "F.Cu") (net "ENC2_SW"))
 (segment (start 73.75 92) (end 73.75 68.67) (width 0.2) (layer "B.Cu") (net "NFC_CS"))
 (segment (start 73.75 68.67) (end 61.43 56.35) (width 0.2) (layer "B.Cu") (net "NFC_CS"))
 (segment (start 71.25 68.71) (end 71.25 92) (width 0.2) (layer "B.Cu") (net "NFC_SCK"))
 (segment (start 61.43 58.89) (end 71.25 68.71) (width 0.2) (layer "B.Cu") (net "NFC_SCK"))
 (segment (start 68.75 68.75) (end 68.75 92) (width 0.2) (layer "B.Cu") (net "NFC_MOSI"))
 (segment (start 61.43 61.43) (end 68.75 68.75) (width 0.2) (layer "B.Cu") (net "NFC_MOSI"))
 (segment (start 66.25 68.79) (end 66.25 92) (width 0.2) (layer "B.Cu") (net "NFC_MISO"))
 (segment (start 61.43 63.97) (end 66.25 68.79) (width 0.2) (layer "B.Cu") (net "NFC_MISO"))
 (segment (start 61.43 66.51) (end 63.75 68.83) (width 0.2) (layer "B.Cu") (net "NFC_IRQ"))
 (segment (start 63.75 68.83) (end 63.75 92) (width 0.2) (layer "B.Cu") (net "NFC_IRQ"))
 (segment (start 58.75 92) (end 59.9017 92) (width 0.2) (layer "B.Cu") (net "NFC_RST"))
 (segment (start 59.9017 90.8483) (end 62.6461 88.1039) (width 0.2) (layer "B.Cu") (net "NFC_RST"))
 (segment (start 62.6461 88.1039) (end 62.6461 70.2661) (width 0.2) (layer "B.Cu") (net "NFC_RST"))
 (segment (start 62.6461 70.2661) (end 61.43 69.05) (width 0.2) (layer "B.Cu") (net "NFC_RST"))
 (segment (start 59.9017 92) (end 59.9017 90.8483) (width 0.2) (layer "B.Cu") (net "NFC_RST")))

